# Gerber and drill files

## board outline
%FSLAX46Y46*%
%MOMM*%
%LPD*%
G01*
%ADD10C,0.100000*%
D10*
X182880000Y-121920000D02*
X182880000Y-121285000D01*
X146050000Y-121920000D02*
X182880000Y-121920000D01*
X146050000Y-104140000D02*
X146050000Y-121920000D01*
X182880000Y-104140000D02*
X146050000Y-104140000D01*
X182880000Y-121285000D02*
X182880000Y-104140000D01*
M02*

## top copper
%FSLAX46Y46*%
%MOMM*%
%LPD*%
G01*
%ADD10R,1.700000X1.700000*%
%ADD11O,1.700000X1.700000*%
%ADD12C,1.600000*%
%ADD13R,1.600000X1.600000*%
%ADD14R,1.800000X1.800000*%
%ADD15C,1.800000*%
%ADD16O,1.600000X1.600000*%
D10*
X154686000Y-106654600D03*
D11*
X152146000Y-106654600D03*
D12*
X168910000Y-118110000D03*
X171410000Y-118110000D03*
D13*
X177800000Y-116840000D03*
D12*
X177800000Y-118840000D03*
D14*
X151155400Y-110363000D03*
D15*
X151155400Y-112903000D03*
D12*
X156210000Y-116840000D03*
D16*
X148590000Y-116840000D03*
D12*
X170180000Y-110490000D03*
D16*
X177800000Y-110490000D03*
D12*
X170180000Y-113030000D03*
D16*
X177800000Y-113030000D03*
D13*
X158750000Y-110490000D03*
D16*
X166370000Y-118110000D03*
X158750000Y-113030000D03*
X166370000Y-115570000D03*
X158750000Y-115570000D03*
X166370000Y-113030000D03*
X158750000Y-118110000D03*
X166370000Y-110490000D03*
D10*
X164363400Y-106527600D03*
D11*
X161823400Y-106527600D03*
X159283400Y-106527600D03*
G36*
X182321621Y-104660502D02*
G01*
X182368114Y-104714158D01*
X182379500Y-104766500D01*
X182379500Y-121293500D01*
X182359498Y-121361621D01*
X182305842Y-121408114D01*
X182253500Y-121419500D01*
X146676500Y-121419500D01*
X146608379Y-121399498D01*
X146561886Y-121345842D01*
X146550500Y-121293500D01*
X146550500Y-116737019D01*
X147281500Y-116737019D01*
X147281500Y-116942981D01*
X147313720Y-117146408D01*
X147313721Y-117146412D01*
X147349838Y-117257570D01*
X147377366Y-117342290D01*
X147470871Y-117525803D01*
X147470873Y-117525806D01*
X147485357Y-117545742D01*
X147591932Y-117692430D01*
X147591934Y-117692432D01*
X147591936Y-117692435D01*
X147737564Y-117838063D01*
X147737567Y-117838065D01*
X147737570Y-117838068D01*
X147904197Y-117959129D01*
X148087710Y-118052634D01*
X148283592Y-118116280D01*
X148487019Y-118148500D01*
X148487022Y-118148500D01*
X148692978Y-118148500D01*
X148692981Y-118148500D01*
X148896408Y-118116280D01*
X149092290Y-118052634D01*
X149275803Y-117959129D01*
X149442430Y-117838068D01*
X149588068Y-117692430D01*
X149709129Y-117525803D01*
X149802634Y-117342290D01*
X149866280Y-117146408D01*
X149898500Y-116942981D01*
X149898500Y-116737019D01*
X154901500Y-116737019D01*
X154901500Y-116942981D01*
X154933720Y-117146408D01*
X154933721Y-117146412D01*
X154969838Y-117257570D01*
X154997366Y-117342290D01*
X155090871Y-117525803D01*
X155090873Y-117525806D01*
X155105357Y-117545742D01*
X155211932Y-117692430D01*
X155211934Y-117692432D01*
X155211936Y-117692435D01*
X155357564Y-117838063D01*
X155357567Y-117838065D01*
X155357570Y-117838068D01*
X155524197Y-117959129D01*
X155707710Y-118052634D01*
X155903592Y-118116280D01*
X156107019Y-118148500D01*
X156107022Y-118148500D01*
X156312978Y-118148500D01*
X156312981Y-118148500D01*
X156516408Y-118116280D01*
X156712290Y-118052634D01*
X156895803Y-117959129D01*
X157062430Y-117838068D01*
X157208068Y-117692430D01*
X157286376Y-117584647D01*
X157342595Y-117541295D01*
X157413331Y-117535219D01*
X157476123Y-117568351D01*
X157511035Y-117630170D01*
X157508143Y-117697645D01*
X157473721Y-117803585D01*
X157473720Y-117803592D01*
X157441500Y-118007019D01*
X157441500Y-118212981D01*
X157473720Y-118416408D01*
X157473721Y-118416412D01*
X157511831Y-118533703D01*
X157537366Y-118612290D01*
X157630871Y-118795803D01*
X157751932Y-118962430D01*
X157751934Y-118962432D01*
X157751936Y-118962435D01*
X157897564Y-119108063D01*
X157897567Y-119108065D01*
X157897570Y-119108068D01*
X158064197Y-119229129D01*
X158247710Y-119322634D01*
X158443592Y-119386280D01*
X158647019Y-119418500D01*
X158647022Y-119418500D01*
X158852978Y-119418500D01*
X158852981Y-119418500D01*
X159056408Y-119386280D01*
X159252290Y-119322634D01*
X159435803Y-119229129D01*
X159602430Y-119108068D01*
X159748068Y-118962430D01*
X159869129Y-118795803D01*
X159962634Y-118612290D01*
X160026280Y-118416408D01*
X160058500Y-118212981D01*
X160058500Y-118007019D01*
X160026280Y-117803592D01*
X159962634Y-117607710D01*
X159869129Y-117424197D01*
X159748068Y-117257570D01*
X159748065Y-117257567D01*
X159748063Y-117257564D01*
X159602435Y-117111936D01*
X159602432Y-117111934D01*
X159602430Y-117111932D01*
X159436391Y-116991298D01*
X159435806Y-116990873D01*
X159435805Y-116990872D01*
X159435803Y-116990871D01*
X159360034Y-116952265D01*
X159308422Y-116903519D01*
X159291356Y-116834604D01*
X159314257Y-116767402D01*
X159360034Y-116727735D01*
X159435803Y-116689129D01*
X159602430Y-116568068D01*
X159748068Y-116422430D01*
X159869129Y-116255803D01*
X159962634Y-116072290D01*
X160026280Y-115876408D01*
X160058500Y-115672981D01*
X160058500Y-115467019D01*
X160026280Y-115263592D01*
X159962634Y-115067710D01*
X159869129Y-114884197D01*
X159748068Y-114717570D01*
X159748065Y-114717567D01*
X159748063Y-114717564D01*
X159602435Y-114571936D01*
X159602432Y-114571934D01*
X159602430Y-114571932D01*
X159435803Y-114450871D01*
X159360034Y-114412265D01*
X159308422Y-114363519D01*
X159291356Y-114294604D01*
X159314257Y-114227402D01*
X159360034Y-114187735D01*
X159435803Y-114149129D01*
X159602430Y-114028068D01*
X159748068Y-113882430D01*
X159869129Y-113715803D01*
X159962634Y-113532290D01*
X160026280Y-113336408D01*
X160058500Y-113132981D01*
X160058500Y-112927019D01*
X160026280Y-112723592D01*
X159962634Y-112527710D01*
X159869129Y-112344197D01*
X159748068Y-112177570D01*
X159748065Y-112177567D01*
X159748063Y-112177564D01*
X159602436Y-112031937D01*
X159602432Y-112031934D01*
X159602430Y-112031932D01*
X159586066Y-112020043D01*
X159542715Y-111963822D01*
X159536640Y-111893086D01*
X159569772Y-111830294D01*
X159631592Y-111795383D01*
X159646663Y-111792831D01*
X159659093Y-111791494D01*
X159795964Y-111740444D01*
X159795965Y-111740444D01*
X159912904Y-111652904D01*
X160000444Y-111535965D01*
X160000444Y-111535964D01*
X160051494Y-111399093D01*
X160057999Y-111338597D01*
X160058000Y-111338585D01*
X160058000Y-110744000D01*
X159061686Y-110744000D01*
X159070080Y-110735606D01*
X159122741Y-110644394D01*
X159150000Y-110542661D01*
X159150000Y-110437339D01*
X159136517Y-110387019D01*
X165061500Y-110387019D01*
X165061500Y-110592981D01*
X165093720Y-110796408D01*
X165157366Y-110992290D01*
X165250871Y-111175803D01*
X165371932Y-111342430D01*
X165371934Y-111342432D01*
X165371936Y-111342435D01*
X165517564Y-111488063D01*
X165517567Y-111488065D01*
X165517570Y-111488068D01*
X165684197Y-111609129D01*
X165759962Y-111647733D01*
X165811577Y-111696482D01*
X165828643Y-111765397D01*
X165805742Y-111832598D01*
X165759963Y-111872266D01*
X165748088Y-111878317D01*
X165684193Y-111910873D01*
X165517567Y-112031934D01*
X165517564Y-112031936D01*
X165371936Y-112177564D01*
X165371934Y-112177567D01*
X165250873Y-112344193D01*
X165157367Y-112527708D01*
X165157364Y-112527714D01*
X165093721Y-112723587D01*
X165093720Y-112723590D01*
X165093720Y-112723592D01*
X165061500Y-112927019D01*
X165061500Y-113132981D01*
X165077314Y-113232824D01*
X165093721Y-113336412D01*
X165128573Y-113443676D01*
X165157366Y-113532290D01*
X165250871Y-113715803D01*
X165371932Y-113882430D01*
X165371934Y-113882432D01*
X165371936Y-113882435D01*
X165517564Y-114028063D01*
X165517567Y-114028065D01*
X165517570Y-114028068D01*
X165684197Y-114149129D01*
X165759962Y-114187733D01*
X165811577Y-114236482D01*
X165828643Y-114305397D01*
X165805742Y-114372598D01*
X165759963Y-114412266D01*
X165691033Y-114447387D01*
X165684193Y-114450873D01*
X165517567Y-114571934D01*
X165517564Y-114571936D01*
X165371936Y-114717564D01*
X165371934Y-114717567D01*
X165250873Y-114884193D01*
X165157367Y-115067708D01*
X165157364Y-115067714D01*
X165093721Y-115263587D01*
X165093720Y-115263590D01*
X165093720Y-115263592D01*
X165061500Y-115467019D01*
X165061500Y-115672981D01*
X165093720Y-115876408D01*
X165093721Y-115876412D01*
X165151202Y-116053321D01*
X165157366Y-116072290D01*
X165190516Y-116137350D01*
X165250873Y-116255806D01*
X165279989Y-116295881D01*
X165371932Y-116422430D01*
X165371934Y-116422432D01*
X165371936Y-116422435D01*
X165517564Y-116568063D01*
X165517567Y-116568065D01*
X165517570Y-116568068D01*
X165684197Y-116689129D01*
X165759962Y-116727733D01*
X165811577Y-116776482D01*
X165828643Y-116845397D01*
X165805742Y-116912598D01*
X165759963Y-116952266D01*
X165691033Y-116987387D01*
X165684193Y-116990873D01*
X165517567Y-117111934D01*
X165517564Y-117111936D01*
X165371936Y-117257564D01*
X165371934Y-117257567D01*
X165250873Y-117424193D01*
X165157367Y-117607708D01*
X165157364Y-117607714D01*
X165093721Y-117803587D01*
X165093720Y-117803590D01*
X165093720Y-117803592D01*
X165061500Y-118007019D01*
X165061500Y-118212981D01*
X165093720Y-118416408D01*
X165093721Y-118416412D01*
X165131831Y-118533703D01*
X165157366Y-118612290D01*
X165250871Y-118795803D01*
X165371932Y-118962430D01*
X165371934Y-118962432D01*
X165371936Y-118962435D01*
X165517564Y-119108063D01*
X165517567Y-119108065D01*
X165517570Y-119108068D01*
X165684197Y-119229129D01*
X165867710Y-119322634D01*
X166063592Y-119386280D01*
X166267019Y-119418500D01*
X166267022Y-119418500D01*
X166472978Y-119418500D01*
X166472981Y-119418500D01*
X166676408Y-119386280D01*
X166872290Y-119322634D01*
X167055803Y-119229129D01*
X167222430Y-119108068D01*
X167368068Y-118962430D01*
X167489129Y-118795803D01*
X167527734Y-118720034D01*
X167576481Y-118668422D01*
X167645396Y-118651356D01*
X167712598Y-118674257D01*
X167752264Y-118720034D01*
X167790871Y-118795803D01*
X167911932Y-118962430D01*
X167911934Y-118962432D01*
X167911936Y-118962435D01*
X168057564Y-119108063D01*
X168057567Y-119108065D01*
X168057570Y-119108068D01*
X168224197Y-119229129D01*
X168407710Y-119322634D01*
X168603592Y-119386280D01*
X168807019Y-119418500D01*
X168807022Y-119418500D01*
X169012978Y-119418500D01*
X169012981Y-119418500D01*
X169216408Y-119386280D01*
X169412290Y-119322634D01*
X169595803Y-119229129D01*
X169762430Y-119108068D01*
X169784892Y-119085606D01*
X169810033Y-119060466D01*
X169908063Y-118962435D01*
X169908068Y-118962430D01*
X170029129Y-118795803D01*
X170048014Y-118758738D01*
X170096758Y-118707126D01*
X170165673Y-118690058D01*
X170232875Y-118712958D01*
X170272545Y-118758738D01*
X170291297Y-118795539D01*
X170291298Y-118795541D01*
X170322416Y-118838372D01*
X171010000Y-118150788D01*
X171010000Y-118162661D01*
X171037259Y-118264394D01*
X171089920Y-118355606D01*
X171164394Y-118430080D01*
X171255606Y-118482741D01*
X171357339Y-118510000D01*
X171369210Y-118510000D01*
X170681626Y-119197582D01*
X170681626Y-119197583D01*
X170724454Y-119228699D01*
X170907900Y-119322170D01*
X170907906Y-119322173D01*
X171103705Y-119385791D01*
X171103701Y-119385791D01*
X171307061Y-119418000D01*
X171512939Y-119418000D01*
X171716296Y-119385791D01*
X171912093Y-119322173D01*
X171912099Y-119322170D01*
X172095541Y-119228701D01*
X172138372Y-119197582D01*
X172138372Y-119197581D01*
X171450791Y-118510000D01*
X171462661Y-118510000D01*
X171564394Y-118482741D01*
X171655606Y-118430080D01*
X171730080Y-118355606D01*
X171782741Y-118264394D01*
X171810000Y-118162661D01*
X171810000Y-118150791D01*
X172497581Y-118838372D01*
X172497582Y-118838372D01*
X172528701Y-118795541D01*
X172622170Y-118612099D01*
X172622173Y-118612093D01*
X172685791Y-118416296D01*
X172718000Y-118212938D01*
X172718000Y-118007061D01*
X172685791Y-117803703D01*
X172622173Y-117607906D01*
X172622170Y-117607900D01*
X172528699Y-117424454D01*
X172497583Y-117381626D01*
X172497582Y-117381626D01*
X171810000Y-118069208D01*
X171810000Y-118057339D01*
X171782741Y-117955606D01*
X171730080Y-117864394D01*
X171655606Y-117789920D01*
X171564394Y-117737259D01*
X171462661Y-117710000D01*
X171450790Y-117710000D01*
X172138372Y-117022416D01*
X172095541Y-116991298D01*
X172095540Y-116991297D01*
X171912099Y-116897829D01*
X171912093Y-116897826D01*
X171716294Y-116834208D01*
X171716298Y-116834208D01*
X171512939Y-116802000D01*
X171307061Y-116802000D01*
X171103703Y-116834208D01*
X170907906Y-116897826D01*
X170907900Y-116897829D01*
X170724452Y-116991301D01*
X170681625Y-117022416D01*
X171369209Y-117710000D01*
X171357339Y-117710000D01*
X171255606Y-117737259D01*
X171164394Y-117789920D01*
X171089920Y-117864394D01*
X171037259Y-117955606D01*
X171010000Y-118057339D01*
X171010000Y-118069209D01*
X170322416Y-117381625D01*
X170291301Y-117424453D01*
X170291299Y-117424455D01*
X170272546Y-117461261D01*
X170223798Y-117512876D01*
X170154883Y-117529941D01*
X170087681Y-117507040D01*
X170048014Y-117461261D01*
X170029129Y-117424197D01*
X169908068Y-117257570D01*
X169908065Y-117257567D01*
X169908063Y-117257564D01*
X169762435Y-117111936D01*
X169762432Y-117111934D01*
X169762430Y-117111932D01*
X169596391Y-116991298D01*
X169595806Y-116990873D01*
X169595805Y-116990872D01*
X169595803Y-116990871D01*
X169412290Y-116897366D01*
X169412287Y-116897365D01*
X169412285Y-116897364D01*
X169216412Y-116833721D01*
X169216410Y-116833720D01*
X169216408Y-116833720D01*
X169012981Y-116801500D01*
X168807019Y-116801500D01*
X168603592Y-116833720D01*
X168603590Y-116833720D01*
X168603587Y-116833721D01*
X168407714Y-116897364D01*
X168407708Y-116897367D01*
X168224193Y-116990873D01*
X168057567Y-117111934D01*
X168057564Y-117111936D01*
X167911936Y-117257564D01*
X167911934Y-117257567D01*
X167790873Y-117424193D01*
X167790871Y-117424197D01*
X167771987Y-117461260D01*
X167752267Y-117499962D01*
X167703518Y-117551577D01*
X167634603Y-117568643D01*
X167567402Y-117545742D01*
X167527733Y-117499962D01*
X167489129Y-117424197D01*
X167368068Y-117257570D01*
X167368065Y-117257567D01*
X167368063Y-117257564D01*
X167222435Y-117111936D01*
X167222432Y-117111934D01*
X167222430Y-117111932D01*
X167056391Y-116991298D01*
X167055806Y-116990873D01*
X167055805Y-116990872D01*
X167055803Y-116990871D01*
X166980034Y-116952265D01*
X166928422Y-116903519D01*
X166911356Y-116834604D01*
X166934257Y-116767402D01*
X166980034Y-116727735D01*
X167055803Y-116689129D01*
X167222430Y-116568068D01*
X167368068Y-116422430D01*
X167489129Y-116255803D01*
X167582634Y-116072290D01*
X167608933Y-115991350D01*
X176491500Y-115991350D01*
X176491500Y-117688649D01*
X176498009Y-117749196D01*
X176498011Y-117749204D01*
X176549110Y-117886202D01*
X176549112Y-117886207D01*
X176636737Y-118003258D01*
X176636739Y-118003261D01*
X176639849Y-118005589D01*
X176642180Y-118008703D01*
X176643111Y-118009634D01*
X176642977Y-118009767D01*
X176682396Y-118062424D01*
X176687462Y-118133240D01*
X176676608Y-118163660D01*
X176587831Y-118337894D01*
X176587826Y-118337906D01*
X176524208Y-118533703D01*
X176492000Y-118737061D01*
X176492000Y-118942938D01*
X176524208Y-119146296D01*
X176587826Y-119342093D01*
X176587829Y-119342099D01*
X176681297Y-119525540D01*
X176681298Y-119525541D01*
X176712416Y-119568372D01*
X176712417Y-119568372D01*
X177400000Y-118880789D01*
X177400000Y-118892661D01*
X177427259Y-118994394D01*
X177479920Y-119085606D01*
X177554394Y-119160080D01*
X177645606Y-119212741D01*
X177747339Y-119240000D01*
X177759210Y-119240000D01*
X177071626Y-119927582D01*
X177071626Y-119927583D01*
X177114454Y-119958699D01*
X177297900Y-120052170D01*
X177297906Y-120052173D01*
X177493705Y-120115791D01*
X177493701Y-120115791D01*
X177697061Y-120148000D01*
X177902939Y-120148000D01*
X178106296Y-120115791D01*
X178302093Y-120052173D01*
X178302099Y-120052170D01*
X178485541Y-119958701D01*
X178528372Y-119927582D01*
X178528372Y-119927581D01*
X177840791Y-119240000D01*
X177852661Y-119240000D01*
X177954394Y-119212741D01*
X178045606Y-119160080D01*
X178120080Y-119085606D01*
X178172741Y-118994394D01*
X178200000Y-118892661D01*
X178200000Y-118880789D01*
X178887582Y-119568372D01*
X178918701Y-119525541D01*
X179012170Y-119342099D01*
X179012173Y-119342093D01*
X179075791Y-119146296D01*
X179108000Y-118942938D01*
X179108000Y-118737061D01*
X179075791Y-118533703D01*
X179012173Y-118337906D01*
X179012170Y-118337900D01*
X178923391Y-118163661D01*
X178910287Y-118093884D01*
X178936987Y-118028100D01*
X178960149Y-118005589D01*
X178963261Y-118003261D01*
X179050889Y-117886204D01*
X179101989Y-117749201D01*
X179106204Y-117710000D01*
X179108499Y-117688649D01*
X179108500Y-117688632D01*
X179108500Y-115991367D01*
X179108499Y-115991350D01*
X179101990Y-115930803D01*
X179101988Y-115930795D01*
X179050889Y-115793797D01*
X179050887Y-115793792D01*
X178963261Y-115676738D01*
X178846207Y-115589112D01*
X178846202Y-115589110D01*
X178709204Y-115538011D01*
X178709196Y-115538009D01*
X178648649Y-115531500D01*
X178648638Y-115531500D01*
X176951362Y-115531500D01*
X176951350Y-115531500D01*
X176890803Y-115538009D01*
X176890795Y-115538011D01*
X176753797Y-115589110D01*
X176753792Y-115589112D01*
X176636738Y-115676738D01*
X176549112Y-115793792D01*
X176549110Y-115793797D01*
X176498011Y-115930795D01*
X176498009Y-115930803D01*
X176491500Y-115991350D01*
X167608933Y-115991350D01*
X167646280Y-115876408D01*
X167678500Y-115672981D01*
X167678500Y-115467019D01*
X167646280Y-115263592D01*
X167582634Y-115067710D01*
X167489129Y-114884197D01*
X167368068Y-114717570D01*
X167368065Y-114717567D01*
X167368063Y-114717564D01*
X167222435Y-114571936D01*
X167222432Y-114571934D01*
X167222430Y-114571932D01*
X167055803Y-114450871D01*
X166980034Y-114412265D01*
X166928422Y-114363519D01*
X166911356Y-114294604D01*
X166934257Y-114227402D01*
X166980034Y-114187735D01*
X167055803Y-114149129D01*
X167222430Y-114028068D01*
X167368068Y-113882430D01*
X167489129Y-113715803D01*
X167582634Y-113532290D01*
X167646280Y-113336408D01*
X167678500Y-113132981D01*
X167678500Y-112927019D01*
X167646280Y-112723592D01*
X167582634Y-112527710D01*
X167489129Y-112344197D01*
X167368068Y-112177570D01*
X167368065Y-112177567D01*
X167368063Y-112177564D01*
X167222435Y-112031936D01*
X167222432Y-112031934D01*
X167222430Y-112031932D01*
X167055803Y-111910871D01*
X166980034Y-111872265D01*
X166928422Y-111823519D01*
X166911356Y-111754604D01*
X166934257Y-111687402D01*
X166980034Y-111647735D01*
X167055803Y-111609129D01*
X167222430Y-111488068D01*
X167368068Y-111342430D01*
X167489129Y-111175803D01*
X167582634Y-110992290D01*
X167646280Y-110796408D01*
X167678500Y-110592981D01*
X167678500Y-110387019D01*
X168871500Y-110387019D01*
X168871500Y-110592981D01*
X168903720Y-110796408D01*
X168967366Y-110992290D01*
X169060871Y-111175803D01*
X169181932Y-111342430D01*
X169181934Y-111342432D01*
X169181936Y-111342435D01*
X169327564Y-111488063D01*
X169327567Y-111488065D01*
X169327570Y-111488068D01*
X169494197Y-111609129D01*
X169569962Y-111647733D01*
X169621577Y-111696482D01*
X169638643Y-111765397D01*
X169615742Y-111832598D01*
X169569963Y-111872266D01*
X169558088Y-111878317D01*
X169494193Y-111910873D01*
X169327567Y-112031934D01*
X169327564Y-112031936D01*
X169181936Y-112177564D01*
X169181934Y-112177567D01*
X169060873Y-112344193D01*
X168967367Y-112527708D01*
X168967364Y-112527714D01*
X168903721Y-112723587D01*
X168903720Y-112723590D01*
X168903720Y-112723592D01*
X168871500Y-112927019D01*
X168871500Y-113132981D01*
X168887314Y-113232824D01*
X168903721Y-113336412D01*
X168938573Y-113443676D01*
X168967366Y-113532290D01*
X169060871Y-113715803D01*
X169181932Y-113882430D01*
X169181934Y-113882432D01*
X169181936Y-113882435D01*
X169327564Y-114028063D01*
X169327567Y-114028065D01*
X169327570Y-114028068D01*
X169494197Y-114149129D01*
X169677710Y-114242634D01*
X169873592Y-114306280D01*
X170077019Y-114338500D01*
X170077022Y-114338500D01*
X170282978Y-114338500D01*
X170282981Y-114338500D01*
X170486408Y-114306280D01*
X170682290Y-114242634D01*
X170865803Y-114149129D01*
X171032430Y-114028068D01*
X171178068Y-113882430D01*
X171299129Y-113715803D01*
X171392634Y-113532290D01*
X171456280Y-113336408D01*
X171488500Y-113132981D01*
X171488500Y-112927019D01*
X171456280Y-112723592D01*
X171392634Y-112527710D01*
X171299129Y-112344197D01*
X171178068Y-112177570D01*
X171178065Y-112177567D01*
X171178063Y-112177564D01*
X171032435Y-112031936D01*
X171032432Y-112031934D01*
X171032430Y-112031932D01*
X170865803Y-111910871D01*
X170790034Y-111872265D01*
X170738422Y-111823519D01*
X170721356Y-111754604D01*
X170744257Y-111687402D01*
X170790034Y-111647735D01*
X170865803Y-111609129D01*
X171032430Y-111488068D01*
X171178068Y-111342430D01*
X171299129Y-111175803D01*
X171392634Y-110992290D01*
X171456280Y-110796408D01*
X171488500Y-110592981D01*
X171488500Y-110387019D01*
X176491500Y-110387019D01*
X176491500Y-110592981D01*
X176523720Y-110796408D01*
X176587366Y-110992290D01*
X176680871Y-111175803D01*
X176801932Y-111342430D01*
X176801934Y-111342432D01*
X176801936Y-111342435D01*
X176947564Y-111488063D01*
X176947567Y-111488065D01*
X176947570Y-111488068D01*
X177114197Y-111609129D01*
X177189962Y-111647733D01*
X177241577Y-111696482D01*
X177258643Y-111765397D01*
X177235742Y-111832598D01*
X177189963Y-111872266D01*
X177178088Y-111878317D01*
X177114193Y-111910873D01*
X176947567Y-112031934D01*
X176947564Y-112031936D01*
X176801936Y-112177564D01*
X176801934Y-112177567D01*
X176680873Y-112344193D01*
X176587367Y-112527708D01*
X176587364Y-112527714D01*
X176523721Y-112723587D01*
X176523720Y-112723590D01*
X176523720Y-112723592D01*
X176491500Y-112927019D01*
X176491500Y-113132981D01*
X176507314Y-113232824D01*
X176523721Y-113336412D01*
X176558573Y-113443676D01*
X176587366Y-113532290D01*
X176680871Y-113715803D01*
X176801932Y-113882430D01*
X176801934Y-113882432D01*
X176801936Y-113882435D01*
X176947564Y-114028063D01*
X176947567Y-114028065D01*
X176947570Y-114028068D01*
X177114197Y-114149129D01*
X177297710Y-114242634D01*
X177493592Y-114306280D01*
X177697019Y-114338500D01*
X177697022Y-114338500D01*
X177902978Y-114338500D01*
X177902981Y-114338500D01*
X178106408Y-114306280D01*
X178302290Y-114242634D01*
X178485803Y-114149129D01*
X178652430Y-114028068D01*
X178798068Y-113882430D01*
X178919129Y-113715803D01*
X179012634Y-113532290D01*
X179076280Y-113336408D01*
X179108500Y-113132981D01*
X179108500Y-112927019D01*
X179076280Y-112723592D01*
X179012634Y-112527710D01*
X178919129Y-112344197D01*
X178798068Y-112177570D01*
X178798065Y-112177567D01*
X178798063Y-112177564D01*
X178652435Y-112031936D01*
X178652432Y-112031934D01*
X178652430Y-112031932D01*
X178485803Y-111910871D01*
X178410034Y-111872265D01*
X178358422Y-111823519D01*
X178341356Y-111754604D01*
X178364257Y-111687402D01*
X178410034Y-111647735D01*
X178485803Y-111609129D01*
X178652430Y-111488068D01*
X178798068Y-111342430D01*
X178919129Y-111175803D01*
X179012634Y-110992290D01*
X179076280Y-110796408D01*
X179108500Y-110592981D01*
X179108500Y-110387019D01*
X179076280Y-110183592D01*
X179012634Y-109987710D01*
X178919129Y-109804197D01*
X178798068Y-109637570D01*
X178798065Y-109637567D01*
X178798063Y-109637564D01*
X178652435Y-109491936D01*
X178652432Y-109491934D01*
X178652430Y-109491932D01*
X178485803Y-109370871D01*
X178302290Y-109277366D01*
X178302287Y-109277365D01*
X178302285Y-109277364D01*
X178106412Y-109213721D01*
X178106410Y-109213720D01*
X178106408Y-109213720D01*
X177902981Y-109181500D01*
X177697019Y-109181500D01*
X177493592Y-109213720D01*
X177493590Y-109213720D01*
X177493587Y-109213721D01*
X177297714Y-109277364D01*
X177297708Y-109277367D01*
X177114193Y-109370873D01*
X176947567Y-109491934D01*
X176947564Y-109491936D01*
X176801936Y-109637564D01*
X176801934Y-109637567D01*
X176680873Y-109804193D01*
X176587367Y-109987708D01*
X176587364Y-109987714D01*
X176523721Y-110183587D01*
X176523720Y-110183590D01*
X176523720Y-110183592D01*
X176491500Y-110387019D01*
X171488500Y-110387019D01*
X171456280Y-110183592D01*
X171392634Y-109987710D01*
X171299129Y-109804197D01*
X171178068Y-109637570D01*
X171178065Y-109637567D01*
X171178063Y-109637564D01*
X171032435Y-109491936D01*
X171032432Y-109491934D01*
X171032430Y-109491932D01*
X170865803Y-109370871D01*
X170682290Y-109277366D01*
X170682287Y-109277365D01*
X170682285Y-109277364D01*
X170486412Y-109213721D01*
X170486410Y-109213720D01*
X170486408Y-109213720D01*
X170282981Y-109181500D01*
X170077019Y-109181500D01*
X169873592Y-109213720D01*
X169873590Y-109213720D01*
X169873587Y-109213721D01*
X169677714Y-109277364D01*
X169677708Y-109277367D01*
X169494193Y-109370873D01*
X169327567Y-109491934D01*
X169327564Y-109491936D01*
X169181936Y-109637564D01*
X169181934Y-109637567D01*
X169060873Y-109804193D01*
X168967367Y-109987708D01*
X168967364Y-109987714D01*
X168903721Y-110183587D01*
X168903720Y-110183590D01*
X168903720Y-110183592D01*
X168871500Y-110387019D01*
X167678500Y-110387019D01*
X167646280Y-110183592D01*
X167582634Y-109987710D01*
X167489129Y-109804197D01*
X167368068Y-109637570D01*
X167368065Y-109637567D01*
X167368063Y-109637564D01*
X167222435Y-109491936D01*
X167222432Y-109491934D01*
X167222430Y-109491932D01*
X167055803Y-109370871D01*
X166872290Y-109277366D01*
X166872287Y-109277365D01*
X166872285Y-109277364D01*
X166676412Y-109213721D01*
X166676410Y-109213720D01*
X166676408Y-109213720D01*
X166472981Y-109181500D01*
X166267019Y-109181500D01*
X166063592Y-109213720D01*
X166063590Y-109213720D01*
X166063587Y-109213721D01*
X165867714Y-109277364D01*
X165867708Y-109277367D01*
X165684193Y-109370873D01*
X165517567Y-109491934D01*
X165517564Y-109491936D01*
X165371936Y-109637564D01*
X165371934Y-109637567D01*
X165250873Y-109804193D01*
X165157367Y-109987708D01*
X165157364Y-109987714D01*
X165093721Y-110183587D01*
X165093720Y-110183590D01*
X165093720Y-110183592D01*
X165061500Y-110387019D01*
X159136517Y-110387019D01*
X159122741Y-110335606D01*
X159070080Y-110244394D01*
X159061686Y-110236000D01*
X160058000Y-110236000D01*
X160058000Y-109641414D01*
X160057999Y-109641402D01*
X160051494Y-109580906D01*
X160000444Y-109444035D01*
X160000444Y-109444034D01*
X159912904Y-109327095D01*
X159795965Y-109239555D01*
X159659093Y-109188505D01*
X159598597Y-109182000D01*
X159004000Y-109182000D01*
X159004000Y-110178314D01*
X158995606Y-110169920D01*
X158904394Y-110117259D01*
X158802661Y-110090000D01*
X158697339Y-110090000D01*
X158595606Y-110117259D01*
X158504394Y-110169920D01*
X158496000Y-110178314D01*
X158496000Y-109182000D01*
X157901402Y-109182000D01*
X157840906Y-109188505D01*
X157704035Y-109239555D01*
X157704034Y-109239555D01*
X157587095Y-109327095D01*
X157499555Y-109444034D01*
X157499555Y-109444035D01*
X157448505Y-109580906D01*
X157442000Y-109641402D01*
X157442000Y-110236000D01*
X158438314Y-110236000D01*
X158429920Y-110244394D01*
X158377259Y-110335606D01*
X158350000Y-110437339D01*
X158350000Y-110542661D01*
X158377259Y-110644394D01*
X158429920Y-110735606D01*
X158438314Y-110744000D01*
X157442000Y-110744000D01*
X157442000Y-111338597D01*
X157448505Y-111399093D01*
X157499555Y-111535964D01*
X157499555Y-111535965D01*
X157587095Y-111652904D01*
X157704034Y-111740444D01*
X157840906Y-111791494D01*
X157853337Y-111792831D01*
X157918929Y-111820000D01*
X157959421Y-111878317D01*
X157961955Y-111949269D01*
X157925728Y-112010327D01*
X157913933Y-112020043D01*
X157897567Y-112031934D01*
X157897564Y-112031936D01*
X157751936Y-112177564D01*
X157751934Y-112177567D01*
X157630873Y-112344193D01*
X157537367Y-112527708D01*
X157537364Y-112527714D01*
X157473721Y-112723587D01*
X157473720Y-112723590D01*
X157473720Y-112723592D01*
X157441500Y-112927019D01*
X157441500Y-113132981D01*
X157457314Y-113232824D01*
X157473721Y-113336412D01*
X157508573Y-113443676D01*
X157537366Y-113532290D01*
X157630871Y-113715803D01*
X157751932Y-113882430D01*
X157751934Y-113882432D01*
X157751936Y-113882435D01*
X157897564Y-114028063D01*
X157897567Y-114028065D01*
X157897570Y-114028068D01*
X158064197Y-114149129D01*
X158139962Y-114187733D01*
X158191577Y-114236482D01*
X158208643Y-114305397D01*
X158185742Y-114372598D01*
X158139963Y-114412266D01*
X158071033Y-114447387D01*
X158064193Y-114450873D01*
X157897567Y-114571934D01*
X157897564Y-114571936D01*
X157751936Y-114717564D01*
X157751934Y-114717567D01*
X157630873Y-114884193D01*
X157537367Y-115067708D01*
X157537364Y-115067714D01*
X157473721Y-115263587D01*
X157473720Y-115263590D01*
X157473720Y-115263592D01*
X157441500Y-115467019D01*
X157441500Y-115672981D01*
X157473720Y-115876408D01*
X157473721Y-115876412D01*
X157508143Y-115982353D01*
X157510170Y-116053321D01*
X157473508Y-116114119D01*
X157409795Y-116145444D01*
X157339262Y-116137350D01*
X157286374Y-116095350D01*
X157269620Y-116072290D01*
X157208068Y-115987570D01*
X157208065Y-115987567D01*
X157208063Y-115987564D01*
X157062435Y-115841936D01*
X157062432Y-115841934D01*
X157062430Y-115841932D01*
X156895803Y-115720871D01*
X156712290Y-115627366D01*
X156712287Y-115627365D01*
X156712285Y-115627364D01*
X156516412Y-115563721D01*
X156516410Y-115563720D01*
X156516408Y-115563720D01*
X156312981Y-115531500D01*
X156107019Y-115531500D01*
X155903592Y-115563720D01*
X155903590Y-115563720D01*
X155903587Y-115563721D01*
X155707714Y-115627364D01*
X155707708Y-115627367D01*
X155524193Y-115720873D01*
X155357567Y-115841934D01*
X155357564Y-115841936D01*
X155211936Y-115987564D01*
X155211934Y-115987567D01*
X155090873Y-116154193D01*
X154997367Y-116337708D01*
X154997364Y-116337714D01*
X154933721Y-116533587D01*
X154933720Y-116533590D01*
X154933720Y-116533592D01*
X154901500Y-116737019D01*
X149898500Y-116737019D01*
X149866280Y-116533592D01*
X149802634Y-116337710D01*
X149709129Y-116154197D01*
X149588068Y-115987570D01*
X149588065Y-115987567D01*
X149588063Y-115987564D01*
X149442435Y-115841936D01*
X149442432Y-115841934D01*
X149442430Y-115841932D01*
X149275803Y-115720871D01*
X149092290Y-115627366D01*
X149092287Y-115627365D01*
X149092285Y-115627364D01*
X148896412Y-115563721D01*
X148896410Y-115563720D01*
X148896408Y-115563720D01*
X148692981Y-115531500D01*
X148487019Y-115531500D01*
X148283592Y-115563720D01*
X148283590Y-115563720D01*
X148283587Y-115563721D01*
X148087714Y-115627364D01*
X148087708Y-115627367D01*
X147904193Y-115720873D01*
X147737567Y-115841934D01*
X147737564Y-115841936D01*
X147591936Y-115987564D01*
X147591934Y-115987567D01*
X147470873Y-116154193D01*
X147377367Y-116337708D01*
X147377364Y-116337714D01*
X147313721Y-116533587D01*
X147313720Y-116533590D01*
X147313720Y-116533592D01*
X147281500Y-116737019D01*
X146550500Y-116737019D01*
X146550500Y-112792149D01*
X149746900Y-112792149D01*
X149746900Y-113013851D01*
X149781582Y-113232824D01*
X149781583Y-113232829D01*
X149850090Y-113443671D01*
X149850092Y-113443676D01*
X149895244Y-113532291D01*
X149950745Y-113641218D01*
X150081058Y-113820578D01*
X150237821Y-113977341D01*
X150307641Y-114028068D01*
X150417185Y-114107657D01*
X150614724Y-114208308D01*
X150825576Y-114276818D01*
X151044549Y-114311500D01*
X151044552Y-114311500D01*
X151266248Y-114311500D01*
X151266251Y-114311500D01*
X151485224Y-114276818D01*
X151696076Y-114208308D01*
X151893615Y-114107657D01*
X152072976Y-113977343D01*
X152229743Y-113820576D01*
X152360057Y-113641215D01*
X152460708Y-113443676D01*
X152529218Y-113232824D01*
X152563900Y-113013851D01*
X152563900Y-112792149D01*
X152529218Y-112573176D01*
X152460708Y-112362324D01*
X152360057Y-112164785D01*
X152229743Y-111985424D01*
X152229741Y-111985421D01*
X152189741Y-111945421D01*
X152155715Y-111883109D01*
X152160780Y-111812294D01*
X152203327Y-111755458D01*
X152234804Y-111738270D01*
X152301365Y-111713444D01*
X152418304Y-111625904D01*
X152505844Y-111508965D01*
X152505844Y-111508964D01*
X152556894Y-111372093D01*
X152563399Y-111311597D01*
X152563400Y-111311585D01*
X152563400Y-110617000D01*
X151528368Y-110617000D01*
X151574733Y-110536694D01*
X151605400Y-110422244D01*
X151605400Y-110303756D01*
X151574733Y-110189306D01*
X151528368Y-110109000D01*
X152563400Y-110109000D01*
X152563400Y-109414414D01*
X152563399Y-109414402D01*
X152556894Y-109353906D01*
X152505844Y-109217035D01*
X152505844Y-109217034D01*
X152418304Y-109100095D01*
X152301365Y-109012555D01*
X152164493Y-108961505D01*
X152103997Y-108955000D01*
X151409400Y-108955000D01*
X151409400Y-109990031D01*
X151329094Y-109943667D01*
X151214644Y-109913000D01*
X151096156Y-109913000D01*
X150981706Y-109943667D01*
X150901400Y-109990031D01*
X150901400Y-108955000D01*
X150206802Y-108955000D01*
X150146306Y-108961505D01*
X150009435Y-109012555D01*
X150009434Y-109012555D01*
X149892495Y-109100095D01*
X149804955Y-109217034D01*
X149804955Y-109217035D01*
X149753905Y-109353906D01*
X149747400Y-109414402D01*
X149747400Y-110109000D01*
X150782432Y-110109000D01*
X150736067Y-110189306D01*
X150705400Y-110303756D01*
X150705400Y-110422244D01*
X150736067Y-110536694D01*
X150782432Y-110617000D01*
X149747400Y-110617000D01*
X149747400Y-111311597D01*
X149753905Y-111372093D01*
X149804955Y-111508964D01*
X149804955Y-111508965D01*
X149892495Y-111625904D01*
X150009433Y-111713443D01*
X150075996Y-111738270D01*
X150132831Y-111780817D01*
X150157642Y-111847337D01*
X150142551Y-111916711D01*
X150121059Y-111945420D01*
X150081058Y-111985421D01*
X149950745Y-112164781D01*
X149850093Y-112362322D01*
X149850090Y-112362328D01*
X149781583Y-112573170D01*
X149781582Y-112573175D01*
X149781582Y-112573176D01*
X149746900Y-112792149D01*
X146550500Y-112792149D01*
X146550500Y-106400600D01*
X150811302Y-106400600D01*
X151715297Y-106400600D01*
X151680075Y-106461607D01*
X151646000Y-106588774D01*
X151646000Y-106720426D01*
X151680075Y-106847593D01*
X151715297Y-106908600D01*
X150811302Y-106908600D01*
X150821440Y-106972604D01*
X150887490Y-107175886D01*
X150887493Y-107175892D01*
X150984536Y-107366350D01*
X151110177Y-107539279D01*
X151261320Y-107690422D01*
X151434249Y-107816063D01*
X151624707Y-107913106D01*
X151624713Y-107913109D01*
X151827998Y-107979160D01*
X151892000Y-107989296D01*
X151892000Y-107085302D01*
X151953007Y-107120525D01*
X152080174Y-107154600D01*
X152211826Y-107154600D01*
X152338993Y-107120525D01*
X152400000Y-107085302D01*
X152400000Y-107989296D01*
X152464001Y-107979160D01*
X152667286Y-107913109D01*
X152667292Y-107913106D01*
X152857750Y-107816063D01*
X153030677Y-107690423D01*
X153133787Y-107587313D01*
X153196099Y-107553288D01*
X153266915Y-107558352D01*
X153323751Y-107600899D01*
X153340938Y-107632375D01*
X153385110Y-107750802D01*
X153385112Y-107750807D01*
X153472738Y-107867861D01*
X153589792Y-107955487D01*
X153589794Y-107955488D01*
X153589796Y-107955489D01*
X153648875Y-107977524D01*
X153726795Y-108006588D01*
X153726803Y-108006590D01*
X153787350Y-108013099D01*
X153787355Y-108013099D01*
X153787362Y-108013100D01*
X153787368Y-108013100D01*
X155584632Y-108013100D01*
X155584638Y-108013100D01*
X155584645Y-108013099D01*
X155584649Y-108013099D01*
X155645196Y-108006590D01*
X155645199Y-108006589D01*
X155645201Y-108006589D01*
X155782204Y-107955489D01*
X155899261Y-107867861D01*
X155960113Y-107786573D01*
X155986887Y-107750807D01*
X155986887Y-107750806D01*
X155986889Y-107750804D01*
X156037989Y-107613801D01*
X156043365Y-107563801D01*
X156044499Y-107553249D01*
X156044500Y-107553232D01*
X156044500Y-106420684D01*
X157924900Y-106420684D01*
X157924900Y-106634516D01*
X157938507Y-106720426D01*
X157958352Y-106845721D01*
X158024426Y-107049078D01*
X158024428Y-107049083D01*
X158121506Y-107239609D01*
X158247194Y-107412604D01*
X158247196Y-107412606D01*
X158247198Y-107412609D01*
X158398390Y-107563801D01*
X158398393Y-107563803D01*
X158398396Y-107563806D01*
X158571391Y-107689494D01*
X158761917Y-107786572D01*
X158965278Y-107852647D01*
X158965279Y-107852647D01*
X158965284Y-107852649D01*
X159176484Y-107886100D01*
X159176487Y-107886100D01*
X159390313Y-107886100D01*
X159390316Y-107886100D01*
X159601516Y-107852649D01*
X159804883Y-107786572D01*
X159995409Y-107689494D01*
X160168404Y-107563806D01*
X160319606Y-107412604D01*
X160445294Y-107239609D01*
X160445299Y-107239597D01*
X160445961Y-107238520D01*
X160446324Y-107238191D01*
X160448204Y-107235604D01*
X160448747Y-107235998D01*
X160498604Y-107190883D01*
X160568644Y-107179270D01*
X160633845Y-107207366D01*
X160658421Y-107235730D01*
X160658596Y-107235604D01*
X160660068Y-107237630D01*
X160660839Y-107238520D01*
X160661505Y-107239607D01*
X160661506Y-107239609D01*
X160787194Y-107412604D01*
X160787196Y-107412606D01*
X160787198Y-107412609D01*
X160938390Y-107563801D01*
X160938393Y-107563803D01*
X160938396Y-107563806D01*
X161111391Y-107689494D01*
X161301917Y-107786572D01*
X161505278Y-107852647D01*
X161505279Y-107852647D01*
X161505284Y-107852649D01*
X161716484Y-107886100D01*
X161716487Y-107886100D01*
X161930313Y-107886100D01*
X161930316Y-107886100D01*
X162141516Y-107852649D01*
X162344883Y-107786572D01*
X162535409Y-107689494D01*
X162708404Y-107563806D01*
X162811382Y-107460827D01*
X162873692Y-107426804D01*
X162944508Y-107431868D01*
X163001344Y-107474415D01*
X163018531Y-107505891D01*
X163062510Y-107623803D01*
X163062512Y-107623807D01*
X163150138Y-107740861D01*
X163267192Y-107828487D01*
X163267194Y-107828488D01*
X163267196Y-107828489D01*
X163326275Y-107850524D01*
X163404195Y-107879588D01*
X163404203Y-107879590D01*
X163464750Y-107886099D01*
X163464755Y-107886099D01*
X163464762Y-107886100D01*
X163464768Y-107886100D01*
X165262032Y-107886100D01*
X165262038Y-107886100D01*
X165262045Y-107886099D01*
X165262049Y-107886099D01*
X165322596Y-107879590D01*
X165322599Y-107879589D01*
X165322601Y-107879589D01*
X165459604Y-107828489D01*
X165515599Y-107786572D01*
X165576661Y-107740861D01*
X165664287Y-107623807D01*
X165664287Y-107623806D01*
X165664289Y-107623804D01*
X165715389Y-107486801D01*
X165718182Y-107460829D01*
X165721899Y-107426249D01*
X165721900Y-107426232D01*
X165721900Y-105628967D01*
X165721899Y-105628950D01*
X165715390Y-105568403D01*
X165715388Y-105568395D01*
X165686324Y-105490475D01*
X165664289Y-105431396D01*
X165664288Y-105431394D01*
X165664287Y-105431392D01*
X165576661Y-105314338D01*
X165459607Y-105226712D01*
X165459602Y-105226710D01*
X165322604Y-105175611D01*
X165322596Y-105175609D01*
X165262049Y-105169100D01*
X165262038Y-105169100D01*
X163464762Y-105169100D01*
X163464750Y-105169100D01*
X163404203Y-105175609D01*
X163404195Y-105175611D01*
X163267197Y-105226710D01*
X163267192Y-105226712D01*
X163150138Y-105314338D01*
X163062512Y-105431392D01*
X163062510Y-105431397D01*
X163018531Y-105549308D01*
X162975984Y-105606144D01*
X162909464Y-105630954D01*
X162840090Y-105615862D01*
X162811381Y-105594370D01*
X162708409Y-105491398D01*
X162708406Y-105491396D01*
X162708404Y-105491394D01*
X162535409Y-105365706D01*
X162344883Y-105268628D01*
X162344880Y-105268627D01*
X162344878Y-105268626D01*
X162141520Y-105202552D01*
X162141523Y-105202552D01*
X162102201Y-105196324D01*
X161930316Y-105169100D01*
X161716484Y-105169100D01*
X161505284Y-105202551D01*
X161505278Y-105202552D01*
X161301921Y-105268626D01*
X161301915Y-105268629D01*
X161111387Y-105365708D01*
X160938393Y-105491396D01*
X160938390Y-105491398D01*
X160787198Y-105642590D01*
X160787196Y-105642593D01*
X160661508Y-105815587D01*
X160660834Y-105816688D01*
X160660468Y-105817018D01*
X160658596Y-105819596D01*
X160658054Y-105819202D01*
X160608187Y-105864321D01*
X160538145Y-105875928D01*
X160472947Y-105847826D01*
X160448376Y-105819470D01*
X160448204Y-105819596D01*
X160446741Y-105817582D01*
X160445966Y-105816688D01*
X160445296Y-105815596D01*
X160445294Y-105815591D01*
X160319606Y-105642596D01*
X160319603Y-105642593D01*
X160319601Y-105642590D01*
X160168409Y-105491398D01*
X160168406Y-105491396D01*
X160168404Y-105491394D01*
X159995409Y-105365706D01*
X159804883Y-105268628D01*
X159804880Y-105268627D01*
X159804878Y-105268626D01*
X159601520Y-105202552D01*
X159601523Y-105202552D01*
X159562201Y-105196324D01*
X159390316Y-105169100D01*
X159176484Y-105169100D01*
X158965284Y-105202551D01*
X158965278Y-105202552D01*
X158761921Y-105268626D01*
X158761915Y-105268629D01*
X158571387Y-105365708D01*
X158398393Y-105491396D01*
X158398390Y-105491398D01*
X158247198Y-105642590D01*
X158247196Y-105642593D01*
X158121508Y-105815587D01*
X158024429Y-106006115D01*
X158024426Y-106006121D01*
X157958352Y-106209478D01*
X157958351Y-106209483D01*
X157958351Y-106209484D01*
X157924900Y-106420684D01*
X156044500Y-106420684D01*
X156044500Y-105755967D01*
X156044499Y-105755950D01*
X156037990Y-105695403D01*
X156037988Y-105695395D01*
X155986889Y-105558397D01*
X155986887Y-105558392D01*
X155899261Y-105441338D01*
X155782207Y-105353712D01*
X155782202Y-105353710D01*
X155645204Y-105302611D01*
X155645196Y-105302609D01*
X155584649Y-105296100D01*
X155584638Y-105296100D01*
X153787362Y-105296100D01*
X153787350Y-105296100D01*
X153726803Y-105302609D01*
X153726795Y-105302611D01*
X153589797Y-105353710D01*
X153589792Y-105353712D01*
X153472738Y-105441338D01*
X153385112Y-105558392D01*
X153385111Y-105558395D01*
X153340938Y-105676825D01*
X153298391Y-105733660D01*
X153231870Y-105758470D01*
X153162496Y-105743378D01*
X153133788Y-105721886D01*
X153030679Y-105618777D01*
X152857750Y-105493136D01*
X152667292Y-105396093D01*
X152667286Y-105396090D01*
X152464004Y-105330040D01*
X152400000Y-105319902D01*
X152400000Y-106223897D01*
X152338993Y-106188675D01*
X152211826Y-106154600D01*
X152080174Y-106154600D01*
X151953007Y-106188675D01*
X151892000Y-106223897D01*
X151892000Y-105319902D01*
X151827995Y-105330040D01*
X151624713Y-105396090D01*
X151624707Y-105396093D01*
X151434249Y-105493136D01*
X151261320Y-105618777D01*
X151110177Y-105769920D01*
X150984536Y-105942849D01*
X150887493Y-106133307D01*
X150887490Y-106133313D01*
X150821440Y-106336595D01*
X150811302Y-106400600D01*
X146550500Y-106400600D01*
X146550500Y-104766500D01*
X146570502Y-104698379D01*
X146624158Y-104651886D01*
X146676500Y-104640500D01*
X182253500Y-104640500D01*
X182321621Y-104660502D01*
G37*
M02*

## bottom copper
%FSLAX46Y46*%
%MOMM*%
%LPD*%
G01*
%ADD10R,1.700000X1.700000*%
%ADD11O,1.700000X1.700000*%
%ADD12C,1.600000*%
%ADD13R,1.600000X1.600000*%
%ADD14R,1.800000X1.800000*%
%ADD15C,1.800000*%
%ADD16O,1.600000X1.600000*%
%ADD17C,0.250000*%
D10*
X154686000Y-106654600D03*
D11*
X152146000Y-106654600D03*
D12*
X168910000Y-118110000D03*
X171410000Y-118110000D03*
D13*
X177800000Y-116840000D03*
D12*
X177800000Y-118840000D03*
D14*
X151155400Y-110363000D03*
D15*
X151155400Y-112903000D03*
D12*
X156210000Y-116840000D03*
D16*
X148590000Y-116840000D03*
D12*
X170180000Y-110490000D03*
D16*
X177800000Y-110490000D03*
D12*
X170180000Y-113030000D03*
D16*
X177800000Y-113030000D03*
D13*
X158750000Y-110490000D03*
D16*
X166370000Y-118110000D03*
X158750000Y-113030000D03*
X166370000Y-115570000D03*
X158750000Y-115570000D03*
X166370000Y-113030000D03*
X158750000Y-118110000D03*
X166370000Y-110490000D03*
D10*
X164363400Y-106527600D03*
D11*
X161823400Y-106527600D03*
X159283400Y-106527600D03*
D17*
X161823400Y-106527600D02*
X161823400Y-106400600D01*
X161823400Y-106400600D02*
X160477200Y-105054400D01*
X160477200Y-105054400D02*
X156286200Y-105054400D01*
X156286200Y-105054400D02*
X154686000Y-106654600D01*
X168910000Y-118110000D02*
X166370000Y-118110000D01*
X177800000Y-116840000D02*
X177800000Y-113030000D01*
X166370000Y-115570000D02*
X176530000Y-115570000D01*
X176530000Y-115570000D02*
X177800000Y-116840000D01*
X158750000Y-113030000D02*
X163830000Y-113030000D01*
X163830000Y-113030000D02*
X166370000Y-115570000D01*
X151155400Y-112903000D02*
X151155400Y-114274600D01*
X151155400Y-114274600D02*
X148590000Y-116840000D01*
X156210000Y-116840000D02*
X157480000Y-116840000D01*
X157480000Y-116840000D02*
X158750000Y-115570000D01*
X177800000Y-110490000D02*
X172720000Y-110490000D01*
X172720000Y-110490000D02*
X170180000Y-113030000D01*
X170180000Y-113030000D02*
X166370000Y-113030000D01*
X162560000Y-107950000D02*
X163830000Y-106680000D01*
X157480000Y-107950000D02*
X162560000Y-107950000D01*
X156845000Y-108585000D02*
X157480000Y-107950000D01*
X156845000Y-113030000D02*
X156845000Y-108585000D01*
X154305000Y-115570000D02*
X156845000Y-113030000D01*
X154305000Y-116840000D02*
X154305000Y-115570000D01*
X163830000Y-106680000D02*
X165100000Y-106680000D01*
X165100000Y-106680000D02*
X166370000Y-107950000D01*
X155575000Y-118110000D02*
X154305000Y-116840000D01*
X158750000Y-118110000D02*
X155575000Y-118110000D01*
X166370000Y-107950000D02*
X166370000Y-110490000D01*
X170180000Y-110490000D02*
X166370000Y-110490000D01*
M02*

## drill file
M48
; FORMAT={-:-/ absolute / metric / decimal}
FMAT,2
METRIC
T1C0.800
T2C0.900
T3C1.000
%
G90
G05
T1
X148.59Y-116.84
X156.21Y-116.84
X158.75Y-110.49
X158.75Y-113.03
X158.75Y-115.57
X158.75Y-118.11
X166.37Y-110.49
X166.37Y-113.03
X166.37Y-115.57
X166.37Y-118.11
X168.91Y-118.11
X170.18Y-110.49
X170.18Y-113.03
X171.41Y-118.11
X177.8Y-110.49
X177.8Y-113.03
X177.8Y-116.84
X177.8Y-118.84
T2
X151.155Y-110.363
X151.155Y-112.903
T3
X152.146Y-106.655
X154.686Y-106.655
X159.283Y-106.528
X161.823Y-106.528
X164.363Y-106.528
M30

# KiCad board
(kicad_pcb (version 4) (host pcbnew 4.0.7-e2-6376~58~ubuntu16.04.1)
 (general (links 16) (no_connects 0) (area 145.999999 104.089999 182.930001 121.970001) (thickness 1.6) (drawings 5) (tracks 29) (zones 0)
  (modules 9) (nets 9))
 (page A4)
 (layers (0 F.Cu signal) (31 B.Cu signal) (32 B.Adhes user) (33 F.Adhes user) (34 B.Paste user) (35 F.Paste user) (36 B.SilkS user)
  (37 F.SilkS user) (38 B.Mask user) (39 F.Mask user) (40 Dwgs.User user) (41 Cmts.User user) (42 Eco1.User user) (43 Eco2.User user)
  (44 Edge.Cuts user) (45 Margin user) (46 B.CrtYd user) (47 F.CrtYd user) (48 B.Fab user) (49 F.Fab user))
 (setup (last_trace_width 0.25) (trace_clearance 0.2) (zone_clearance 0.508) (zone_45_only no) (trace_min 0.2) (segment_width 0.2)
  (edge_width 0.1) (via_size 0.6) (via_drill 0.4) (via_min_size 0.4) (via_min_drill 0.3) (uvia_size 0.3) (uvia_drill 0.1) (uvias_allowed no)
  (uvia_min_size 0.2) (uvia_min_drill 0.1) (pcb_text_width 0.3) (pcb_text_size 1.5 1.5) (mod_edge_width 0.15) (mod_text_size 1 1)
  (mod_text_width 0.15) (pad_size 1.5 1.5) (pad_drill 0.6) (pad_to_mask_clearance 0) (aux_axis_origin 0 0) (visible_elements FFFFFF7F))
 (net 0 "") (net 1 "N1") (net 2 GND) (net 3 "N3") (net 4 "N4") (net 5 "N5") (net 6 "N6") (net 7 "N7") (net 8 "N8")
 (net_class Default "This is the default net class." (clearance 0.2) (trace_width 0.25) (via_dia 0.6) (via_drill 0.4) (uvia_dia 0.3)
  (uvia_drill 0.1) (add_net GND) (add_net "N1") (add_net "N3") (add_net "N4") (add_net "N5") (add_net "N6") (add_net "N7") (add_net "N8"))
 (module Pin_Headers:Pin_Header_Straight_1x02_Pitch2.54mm (layer F.Cu) (at 154.686 106.6546 270)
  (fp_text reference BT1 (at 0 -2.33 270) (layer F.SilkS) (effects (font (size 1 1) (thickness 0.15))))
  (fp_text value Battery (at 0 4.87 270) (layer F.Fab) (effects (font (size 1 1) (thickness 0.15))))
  (pad 1 thru_hole rect (at 0 0 270) (size 1.7 1.7) (drill 1) (layers *.Cu *.Mask) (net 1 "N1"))
  (pad 2 thru_hole oval (at 0 2.54 270) (size 1.7 1.7) (drill 1) (layers *.Cu *.Mask) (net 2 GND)))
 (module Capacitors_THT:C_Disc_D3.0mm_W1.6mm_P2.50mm (layer F.Cu) (at 168.91 118.11)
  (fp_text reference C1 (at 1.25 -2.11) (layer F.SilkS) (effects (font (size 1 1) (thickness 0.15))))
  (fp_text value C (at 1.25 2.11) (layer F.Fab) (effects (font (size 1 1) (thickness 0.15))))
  (pad 1 thru_hole circle (at 0 0) (size 1.6 1.6) (drill 0.8) (layers *.Cu *.Mask) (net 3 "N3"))
  (pad 2 thru_hole circle (at 2.5 0) (size 1.6 1.6) (drill 0.8) (layers *.Cu *.Mask) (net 2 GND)))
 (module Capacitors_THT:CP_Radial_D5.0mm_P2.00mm (layer F.Cu) (at 177.8 116.84 270)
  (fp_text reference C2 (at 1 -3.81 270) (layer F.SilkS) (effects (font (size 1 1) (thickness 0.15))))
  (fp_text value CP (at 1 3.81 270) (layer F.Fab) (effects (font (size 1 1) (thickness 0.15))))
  (pad 1 thru_hole rect (at 0 0 270) (size 1.6 1.6) (drill 0.8) (layers *.Cu *.Mask) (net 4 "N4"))
  (pad 2 thru_hole circle (at 2 0 270) (size 1.6 1.6) (drill 0.8) (layers *.Cu *.Mask) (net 2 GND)))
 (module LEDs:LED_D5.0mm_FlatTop (layer F.Cu) (at 151.1554 110.363 270)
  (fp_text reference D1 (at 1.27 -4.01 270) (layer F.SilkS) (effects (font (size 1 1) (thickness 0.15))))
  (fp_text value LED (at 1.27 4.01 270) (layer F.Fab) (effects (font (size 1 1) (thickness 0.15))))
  (pad 1 thru_hole rect (at 0 0 270) (size 1.8 1.8) (drill 0.9) (layers *.Cu *.Mask) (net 2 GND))
  (pad 2 thru_hole circle (at 2.54 0 270) (size 1.8 1.8) (drill 0.9) (layers *.Cu *.Mask) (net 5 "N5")))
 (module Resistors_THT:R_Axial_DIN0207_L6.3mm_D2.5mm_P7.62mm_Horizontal (layer F.Cu) (at 156.21 116.84 180)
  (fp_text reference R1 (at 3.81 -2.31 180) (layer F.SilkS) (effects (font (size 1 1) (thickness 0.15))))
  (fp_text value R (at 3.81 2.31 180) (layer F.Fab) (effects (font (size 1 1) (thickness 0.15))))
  (pad 1 thru_hole circle (at 0 0 180) (size 1.6 1.6) (drill 0.8) (layers *.Cu *.Mask) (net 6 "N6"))
  (pad 2 thru_hole oval (at 7.62 0 180) (size 1.6 1.6) (drill 0.8) (layers *.Cu *.Mask) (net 5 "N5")))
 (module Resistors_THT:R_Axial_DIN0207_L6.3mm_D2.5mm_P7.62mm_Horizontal (layer F.Cu) (at 170.18 110.49)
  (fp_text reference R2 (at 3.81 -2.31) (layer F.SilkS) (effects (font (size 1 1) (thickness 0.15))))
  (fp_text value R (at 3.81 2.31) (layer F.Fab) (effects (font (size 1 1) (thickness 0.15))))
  (pad 1 thru_hole circle (at 0 0) (size 1.6 1.6) (drill 0.8) (layers *.Cu *.Mask) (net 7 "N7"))
  (pad 2 thru_hole oval (at 7.62 0) (size 1.6 1.6) (drill 0.8) (layers *.Cu *.Mask) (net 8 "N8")))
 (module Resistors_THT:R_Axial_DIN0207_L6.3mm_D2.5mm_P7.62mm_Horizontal (layer F.Cu) (at 170.18 113.03)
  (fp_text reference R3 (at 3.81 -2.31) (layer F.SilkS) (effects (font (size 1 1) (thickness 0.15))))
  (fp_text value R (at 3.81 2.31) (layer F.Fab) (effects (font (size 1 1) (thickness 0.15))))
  (pad 1 thru_hole circle (at 0 0) (size 1.6 1.6) (drill 0.8) (layers *.Cu *.Mask) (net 8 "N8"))
  (pad 2 thru_hole oval (at 7.62 0) (size 1.6 1.6) (drill 0.8) (layers *.Cu *.Mask) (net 4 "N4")))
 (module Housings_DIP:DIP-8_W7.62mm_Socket (layer F.Cu) (at 158.75 110.49)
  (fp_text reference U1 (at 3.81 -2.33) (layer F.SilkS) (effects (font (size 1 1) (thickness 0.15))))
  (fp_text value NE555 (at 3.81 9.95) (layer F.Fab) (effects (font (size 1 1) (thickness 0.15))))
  (pad 1 thru_hole rect (at 0 0) (size 1.6 1.6) (drill 0.8) (layers *.Cu *.Mask) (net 2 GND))
  (pad 5 thru_hole oval (at 7.62 7.62) (size 1.6 1.6) (drill 0.8) (layers *.Cu *.Mask) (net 3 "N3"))
  (pad 2 thru_hole oval (at 0 2.54) (size 1.6 1.6) (drill 0.8) (layers *.Cu *.Mask) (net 4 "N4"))
  (pad 6 thru_hole oval (at 7.62 5.08) (size 1.6 1.6) (drill 0.8) (layers *.Cu *.Mask) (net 4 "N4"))
  (pad 3 thru_hole oval (at 0 5.08) (size 1.6 1.6) (drill 0.8) (layers *.Cu *.Mask) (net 6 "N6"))
  (pad 7 thru_hole oval (at 7.62 2.54) (size 1.6 1.6) (drill 0.8) (layers *.Cu *.Mask) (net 8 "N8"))
  (pad 4 thru_hole oval (at 0 7.62) (size 1.6 1.6) (drill 0.8) (layers *.Cu *.Mask) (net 7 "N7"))
  (pad 8 thru_hole oval (at 7.62 0) (size 1.6 1.6) (drill 0.8) (layers *.Cu *.Mask) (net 7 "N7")))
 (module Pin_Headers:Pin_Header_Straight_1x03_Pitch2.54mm (layer F.Cu) (at 164.3634 106.5276 270)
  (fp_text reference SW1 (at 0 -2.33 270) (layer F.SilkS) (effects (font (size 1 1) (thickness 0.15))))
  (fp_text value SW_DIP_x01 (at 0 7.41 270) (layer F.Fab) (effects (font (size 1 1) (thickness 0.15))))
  (pad 1 thru_hole rect (at 0 0 270) (size 1.7 1.7) (drill 1) (layers *.Cu *.Mask) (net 7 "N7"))
  (pad 2 thru_hole oval (at 0 2.54 270) (size 1.7 1.7) (drill 1) (layers *.Cu *.Mask) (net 1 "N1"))
  (pad 3 thru_hole oval (at 0 5.08 270) (size 1.7 1.7) (drill 1) (layers *.Cu *.Mask)))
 (gr_line (start 182.88 121.92) (end 182.88 121.285) (angle 90) (layer Edge.Cuts) (width 0.1))
 (gr_line (start 146.05 121.92) (end 182.88 121.92) (angle 90) (layer Edge.Cuts) (width 0.1))
 (gr_line (start 146.05 104.14) (end 146.05 121.92) (angle 90) (layer Edge.Cuts) (width 0.1))
 (gr_line (start 182.88 104.14) (end 146.05 104.14) (angle 90) (layer Edge.Cuts) (width 0.1))
 (gr_line (start 182.88 121.285) (end 182.88 104.14) (angle 90) (layer Edge.Cuts) (width 0.1))
 (segment (start 161.8234 106.5276) (end 161.8234 106.4006) (width 0.25) (layer B.Cu) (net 1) (status C00000))
 (segment (start 161.8234 106.4006) (end 160.4772 105.0544) (width 0.25) (layer B.Cu) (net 1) (status 400000))
 (segment (start 160.4772 105.0544) (end 156.2862 105.0544) (width 0.25) (layer B.Cu) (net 1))
 (segment (start 156.2862 105.0544) (end 154.686 106.6546) (width 0.25) (layer B.Cu) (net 1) (status 800000))
 (segment (start 168.91 118.11) (end 166.37 118.11) (width 0.25) (layer B.Cu) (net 3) (status C00000))
 (segment (start 177.8 116.84) (end 177.8 113.03) (width 0.25) (layer B.Cu) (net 4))
 (segment (start 166.37 115.57) (end 176.53 115.57) (width 0.25) (layer B.Cu) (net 4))
 (segment (start 176.53 115.57) (end 177.8 116.84) (width 0.25) (layer B.Cu) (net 4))
 (segment (start 158.75 113.03) (end 163.83 113.03) (width 0.25) (layer B.Cu) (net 4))
 (segment (start 163.83 113.03) (end 166.37 115.57) (width 0.25) (layer B.Cu) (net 4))
 (segment (start 151.1554 112.903) (end 151.1554 114.2746) (width 0.25) (layer B.Cu) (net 5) (status 400000))
 (segment (start 151.1554 114.2746) (end 148.59 116.84) (width 0.25) (layer B.Cu) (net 5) (status 800000))
 (segment (start 156.21 116.84) (end 157.48 116.84) (width 0.25) (layer B.Cu) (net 6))
 (segment (start 157.48 116.84) (end 158.75 115.57) (width 0.25) (layer B.Cu) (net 6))
 (segment (start 177.8 110.49) (end 172.72 110.49) (width 0.25) (layer B.Cu) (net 8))
 (segment (start 172.72 110.49) (end 170.18 113.03) (width 0.25) (layer B.Cu) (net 8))
 (segment (start 170.18 113.03) (end 166.37 113.03) (width 0.25) (layer B.Cu) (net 8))
 (segment (start 162.56 107.95) (end 163.83 106.68) (width 0.25) (layer B.Cu) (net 7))
 (segment (start 157.48 107.95) (end 162.56 107.95) (width 0.25) (layer B.Cu) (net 7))
 (segment (start 156.845 108.585) (end 157.48 107.95) (width 0.25) (layer B.Cu) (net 7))
 (segment (start 156.845 113.03) (end 156.845 108.585) (width 0.25) (layer B.Cu) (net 7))
 (segment (start 154.305 115.57) (end 156.845 113.03) (width 0.25) (layer B.Cu) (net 7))
 (segment (start 154.305 116.84) (end 154.305 115.57) (width 0.25) (layer B.Cu) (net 7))
 (segment (start 163.83 106.68) (end 165.1 106.68) (width 0.25) (layer B.Cu) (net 7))
 (segment (start 165.1 106.68) (end 166.37 107.95) (width 0.25) (layer B.Cu) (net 7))
 (segment (start 155.575 118.11) (end 154.305 116.84) (width 0.25) (layer B.Cu) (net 7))
 (segment (start 158.75 118.11) (end 155.575 118.11) (width 0.25) (layer B.Cu) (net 7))
 (segment (start 166.37 107.95) (end 166.37 110.49) (width 0.25) (layer B.Cu) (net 7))
 (segment (start 170.18 110.49) (end 166.37 110.49) (width 0.25) (layer B.Cu) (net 7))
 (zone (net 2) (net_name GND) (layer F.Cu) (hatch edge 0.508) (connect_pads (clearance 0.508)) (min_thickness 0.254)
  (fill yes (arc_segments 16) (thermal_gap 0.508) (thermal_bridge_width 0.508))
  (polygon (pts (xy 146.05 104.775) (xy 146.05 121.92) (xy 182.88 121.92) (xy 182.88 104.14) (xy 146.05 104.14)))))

